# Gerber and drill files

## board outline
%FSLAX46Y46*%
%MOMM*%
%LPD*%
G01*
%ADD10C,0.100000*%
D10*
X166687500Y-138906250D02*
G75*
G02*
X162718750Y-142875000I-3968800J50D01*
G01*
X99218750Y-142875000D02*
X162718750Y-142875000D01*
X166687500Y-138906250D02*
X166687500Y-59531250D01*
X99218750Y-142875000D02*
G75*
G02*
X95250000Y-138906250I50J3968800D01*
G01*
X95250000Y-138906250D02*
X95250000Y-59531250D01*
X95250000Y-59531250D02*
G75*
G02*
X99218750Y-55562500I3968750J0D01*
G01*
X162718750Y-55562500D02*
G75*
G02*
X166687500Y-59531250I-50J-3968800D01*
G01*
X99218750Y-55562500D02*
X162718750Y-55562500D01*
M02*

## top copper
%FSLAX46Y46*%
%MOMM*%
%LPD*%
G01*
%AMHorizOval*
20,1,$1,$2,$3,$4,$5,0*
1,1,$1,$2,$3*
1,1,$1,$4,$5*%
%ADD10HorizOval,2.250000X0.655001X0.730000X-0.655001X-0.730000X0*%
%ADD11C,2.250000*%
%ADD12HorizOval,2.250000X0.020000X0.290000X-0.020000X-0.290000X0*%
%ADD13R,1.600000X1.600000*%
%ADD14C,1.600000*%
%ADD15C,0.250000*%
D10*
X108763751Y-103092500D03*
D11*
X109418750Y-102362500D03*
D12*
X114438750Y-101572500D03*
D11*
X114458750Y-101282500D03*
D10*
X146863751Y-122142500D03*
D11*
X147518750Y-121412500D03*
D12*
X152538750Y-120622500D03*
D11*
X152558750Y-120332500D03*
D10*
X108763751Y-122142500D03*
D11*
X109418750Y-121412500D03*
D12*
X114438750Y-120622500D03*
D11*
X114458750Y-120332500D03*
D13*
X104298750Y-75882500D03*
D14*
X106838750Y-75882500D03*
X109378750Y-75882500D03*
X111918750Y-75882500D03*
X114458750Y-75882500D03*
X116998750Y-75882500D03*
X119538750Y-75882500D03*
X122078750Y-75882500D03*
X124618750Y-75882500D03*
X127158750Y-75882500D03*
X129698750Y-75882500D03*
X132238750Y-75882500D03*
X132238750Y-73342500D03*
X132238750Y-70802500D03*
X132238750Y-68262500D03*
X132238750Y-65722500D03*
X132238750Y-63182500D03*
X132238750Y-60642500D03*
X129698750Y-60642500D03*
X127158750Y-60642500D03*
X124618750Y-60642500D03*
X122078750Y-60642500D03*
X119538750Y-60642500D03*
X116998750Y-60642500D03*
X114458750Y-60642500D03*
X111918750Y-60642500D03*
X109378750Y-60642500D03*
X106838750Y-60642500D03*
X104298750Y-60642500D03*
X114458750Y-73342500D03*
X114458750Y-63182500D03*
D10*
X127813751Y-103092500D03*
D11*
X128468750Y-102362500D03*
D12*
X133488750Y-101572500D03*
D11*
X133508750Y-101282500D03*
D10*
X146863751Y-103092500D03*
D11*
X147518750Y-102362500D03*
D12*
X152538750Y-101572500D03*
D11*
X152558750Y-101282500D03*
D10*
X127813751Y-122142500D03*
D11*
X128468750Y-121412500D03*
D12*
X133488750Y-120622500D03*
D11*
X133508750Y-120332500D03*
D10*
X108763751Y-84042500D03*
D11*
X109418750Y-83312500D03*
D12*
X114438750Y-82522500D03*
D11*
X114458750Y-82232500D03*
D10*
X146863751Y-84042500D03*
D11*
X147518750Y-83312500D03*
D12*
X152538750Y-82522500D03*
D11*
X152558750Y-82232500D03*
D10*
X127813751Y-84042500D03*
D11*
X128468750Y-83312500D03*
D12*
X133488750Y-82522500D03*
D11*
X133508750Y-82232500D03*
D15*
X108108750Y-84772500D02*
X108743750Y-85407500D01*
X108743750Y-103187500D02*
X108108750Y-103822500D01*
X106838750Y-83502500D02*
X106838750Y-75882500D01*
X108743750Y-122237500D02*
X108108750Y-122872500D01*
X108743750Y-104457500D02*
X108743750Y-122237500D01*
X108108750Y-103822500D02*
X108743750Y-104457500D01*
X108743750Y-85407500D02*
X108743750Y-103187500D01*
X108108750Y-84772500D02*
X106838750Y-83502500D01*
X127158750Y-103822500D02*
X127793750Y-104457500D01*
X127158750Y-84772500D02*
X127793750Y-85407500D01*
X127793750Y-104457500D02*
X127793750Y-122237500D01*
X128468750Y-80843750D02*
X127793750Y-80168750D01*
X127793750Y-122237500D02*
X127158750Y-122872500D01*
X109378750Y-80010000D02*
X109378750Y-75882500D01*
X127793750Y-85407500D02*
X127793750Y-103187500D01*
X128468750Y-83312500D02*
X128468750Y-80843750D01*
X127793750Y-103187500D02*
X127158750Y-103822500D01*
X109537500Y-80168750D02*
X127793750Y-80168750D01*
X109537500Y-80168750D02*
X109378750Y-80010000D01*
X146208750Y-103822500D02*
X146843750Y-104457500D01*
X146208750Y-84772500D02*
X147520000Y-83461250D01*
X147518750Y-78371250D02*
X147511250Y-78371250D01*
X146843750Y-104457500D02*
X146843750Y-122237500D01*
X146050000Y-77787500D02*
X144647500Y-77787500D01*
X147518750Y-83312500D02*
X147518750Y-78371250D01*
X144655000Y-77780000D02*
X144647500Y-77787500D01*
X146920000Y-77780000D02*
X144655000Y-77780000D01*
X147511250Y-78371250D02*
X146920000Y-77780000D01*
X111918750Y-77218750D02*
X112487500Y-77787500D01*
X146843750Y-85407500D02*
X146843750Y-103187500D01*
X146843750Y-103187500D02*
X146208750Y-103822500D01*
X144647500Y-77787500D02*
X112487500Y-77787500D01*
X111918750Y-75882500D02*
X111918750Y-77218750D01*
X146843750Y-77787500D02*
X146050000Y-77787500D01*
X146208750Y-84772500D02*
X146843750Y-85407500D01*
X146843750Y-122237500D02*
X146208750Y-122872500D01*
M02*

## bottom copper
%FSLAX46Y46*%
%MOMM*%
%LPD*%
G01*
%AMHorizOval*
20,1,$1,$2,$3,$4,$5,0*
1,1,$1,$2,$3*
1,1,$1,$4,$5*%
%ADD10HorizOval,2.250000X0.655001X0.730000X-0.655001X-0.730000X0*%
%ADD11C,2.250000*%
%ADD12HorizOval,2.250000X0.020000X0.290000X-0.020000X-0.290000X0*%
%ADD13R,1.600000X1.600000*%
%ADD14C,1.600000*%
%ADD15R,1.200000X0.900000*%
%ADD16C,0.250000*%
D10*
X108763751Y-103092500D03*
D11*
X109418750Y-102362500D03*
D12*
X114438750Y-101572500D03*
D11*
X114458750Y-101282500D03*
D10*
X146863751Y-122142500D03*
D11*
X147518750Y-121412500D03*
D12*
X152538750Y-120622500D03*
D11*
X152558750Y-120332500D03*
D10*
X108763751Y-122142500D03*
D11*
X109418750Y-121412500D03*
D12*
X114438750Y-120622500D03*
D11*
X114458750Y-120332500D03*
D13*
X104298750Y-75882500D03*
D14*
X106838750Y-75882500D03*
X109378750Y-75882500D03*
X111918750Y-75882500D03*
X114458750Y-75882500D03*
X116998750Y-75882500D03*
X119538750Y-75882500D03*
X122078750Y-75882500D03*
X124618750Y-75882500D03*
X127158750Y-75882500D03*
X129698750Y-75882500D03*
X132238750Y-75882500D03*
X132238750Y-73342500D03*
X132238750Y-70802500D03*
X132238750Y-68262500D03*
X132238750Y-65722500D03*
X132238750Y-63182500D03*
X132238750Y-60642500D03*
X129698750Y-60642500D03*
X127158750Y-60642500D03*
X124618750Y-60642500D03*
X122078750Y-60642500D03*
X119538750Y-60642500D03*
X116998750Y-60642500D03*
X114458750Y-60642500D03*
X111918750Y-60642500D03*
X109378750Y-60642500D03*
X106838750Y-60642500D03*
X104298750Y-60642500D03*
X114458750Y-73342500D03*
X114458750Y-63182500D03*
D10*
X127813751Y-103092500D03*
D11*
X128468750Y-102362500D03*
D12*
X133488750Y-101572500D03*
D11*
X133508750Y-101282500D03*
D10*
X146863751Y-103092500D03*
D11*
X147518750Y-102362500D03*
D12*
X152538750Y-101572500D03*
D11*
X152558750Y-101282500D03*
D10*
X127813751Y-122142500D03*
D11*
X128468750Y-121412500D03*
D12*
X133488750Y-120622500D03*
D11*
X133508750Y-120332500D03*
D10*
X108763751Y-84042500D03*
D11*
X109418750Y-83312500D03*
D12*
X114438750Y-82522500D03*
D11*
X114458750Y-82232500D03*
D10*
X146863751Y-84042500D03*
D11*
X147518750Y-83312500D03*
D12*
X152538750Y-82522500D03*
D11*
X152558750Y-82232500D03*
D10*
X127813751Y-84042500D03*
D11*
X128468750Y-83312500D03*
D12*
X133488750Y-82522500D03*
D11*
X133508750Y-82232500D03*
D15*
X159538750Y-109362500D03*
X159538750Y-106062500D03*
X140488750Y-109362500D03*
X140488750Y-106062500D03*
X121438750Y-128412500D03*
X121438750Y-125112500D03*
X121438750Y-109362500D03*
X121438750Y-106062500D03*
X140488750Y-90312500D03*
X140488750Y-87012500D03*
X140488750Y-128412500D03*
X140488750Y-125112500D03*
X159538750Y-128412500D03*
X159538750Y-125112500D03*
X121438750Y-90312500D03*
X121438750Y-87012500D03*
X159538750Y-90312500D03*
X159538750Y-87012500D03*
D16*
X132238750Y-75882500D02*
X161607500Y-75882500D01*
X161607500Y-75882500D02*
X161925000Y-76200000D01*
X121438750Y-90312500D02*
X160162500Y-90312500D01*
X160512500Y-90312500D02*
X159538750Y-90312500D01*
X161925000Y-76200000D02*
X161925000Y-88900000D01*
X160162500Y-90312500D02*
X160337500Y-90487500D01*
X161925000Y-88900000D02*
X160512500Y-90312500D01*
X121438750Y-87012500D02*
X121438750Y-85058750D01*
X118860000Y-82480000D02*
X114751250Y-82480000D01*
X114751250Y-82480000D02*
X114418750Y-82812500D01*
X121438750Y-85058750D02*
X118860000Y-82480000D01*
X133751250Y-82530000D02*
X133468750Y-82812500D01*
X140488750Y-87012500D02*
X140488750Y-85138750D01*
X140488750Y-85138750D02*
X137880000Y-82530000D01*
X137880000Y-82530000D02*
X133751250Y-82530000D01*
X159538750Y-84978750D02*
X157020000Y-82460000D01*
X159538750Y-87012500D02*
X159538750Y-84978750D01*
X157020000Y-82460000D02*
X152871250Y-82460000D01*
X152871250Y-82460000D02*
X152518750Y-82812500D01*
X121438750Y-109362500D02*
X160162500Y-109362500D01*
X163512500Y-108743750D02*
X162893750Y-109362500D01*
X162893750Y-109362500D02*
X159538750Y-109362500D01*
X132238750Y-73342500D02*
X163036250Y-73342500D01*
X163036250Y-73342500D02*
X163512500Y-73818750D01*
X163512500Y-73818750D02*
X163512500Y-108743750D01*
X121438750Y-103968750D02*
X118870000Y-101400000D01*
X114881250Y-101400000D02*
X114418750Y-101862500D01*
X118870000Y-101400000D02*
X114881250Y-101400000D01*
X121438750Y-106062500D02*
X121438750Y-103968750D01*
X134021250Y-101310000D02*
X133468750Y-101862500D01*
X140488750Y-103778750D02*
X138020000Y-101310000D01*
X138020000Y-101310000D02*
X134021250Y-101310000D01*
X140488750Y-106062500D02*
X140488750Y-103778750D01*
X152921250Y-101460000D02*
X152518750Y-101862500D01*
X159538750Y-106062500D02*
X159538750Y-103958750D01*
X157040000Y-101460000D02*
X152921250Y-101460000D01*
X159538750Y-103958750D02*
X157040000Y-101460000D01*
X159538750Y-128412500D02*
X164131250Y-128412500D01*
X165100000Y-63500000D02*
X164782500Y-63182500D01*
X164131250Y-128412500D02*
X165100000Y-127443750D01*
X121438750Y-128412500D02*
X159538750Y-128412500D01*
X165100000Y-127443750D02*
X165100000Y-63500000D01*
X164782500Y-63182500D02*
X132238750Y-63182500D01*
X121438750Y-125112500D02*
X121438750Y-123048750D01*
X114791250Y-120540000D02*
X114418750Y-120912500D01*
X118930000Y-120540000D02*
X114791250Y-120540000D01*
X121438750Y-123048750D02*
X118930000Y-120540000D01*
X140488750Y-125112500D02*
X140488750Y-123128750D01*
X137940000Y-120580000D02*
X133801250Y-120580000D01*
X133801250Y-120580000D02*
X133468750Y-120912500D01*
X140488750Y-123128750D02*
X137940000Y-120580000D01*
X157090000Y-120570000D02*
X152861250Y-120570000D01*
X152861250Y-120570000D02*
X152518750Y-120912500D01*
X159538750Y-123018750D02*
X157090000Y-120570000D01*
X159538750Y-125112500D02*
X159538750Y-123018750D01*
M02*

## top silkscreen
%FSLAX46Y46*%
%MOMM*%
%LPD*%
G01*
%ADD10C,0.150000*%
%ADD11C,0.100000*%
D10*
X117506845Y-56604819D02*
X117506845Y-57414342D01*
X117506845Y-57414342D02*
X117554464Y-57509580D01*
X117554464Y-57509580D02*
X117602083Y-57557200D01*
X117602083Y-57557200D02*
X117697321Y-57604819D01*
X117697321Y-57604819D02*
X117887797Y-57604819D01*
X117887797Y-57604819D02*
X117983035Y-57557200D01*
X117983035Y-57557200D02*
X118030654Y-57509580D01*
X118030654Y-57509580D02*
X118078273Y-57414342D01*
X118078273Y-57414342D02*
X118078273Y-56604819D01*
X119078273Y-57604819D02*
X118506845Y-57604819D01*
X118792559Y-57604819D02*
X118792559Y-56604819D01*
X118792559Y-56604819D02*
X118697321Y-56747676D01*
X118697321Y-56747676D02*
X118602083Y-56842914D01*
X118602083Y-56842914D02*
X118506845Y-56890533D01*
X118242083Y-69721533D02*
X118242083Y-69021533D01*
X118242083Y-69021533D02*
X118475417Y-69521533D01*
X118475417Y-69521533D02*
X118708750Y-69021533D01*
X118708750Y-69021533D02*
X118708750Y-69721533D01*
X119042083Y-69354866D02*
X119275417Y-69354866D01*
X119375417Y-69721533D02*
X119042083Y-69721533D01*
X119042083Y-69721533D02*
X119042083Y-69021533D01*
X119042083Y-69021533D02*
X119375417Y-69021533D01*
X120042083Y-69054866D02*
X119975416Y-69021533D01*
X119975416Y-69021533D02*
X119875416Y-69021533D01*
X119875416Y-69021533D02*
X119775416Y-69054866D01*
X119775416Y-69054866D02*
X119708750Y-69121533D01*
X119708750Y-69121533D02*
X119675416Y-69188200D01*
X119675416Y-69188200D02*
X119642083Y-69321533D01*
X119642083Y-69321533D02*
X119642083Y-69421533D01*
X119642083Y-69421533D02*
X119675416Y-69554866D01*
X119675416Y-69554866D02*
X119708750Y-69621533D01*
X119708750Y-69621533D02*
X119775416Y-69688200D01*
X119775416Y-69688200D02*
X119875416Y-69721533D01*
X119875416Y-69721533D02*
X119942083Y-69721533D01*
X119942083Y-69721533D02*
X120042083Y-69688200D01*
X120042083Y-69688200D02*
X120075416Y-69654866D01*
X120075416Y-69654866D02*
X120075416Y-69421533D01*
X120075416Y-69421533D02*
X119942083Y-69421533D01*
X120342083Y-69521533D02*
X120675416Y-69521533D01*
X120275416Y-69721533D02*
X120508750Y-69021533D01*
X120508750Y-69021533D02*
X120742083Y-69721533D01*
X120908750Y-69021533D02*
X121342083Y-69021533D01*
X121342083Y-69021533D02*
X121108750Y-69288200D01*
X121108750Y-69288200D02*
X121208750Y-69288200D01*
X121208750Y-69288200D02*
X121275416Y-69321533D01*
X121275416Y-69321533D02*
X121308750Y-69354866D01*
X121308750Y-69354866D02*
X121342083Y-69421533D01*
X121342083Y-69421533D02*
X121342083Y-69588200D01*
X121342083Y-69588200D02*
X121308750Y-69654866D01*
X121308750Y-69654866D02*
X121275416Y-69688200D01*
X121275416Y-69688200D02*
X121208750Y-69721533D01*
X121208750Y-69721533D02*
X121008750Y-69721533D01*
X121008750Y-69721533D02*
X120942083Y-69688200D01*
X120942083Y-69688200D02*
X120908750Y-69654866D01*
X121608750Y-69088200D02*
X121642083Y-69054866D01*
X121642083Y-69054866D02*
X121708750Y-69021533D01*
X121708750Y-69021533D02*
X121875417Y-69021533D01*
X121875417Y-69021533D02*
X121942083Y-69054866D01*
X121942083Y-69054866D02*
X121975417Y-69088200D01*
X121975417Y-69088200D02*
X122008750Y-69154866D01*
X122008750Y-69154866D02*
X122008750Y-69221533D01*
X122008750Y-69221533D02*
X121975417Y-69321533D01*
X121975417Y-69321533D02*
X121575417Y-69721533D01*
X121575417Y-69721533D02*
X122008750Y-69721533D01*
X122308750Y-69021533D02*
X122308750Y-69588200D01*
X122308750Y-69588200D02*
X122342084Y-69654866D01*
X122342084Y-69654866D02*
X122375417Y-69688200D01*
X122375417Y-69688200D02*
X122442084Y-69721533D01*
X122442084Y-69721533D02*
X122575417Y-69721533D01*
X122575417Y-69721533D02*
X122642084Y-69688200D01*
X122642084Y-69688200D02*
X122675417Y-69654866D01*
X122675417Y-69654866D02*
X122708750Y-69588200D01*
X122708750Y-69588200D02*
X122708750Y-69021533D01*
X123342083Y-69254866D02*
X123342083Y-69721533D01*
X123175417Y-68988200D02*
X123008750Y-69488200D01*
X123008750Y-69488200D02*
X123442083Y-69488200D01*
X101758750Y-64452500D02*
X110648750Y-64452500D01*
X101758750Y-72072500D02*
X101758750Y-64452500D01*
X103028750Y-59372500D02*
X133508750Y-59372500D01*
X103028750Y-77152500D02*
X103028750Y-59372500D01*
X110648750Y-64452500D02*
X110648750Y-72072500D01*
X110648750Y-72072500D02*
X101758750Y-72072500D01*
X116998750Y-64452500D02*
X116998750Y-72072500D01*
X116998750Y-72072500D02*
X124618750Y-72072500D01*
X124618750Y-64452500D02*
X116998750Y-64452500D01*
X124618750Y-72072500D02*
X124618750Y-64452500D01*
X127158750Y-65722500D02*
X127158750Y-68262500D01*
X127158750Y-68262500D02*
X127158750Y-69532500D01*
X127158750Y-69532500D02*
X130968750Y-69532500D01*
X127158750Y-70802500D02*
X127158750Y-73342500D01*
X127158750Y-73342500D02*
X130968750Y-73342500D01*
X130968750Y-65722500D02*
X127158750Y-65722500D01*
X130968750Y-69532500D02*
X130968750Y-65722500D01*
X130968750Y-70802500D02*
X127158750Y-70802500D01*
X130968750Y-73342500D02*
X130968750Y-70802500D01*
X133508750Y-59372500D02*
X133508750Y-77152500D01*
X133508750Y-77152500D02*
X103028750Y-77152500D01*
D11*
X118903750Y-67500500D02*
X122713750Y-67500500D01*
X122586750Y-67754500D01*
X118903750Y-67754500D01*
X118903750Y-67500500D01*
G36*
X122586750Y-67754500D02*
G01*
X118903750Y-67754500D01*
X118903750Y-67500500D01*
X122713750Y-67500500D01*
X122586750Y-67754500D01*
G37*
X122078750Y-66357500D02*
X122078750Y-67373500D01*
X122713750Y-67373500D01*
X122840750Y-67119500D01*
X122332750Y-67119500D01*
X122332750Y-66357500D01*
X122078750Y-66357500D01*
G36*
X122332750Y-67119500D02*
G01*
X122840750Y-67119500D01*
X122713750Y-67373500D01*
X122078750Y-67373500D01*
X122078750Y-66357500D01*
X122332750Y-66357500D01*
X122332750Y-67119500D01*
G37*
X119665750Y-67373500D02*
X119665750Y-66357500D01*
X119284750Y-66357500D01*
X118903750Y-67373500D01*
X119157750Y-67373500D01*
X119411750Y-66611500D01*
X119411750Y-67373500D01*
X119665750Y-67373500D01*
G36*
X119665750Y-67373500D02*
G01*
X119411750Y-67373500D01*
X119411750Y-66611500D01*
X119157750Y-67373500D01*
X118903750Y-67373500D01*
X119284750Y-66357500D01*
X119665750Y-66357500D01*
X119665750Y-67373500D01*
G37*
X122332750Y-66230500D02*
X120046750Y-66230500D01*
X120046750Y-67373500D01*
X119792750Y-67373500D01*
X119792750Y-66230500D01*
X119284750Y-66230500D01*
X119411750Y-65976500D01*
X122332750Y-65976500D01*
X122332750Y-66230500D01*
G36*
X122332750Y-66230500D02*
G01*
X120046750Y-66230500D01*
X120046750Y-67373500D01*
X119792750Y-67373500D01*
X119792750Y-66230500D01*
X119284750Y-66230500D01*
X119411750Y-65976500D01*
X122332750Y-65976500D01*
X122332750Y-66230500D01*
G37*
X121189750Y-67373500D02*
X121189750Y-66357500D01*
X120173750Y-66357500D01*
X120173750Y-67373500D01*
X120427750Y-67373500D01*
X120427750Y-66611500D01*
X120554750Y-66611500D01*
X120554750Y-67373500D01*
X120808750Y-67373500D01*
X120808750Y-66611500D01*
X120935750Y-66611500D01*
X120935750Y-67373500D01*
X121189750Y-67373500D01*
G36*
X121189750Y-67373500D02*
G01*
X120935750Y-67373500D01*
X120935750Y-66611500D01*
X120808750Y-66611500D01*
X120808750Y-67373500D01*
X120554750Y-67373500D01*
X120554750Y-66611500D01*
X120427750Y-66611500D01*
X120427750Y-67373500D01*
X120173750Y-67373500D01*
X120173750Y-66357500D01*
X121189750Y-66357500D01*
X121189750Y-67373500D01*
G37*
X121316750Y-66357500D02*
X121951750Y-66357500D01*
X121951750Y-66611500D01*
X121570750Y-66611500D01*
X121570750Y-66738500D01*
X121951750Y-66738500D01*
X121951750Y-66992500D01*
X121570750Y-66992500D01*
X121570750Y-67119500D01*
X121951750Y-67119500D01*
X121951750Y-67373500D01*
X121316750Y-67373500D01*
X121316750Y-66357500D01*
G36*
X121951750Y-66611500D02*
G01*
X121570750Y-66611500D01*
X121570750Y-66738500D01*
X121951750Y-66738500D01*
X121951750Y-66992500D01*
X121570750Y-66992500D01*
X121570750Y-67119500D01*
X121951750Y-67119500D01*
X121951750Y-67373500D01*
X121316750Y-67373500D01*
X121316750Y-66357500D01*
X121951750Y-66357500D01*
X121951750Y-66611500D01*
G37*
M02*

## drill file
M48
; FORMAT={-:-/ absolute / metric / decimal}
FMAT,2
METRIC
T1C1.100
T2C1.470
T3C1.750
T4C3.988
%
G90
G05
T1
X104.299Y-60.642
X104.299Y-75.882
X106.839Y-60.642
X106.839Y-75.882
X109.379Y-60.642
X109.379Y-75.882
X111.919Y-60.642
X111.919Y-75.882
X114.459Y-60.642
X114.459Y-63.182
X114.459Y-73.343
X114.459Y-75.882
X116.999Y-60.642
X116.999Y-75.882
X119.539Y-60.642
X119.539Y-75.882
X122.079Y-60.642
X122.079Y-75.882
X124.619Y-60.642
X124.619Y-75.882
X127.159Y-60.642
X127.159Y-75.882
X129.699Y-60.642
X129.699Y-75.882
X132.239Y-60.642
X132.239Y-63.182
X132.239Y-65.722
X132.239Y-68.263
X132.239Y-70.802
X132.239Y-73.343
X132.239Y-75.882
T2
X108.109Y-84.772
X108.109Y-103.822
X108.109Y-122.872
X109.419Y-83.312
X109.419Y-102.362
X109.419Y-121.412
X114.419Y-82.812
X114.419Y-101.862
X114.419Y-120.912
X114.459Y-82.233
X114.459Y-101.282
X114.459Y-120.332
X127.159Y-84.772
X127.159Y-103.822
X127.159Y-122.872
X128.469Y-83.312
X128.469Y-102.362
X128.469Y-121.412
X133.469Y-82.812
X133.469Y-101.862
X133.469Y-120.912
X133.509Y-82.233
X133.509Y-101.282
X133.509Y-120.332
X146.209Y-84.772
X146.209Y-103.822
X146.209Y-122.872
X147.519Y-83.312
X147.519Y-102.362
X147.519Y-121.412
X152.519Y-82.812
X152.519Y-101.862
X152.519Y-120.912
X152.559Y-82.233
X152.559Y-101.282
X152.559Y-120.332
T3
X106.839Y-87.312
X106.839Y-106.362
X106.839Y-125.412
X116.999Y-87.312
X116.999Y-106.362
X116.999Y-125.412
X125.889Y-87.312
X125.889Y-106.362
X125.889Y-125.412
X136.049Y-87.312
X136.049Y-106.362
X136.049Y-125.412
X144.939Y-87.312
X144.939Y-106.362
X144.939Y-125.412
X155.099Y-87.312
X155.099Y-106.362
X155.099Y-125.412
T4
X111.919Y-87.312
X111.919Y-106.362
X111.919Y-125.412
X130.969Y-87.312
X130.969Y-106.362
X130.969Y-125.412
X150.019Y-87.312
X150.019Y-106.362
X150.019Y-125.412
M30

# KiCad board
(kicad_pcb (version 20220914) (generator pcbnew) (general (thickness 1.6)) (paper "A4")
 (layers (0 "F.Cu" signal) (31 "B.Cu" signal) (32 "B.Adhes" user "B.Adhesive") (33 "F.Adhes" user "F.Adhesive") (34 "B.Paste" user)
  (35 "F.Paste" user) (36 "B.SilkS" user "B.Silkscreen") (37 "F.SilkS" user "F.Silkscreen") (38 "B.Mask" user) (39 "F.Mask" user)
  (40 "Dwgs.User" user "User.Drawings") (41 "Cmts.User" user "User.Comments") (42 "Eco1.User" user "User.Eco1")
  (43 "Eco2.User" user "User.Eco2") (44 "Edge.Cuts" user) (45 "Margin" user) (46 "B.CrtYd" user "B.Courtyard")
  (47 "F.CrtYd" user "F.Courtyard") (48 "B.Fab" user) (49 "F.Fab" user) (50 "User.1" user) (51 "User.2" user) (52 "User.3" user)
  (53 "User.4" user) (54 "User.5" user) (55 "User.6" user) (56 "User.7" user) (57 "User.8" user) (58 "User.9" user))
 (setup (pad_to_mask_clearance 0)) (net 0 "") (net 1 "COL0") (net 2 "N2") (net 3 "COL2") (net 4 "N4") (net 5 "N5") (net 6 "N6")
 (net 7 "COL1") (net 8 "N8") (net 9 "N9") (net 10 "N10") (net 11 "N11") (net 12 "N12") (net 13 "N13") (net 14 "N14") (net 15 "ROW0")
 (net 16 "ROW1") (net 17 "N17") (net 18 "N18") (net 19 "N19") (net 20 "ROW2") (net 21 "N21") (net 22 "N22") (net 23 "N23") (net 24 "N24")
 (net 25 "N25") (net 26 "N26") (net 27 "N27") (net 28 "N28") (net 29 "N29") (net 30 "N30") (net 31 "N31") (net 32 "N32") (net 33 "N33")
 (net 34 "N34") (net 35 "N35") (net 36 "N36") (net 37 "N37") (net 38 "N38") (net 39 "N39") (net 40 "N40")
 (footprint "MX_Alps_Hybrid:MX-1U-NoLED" (layer "F.Cu") (at 111.91875 106.3625)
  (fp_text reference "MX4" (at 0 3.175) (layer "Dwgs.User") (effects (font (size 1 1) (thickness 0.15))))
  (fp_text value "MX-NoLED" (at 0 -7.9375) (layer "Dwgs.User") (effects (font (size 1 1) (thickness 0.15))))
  (pad "" np_thru_hole circle (at -5.08 0 48.0996) (size 1.75 1.75) (drill 1.75) (layers *.Cu *.Mask))
  (pad "" np_thru_hole circle (at 0 0) (size 3.9878 3.9878) (drill 3.9878) (layers *.Cu *.Mask))
  (pad "" np_thru_hole circle (at 5.08 0 48.0996) (size 1.75 1.75) (drill 1.75) (layers *.Cu *.Mask))
  (pad "1" thru_hole oval (at -3.81 -2.54 48.0996) (size 4.211556 2.25) (drill 1.47 (offset 0.980778 0)) (layers *.Cu "B.Mask")
   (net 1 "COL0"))
  (pad "1" thru_hole circle (at -2.5 -4) (size 2.25 2.25) (drill 1.47) (layers *.Cu "B.Mask") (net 1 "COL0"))
  (pad "2" thru_hole oval (at 2.5 -4.5 86.0548) (size 2.831378 2.25) (drill 1.47 (offset 0.290689 0)) (layers *.Cu "B.Mask") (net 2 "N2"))
  (pad "2" thru_hole circle (at 2.54 -5.08) (size 2.25 2.25) (drill 1.47) (layers *.Cu "B.Mask") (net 2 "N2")))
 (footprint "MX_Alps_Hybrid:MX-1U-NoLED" (layer "F.Cu") (at 150.01875 125.4125)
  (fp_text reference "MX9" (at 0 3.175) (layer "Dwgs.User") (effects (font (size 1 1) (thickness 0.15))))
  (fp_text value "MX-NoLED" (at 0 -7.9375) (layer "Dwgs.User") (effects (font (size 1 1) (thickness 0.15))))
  (pad "" np_thru_hole circle (at -5.08 0 48.0996) (size 1.75 1.75) (drill 1.75) (layers *.Cu *.Mask))
  (pad "" np_thru_hole circle (at 0 0) (size 3.9878 3.9878) (drill 3.9878) (layers *.Cu *.Mask))
  (pad "" np_thru_hole circle (at 5.08 0 48.0996) (size 1.75 1.75) (drill 1.75) (layers *.Cu *.Mask))
  (pad "1" thru_hole oval (at -3.81 -2.54 48.0996) (size 4.211556 2.25) (drill 1.47 (offset 0.980778 0)) (layers *.Cu "B.Mask")
   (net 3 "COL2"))
  (pad "1" thru_hole circle (at -2.5 -4) (size 2.25 2.25) (drill 1.47) (layers *.Cu "B.Mask") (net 3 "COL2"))
  (pad "2" thru_hole oval (at 2.5 -4.5 86.0548) (size 2.831378 2.25) (drill 1.47 (offset 0.290689 0)) (layers *.Cu "B.Mask") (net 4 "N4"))
  (pad "2" thru_hole circle (at 2.54 -5.08) (size 2.25 2.25) (drill 1.47) (layers *.Cu "B.Mask") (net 4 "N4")))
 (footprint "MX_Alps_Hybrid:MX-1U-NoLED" (layer "F.Cu") (at 111.91875 125.4125)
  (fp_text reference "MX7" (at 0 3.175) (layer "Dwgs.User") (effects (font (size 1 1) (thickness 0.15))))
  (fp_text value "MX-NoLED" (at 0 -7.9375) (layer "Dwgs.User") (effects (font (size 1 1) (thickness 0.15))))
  (pad "" np_thru_hole circle (at -5.08 0 48.0996) (size 1.75 1.75) (drill 1.75) (layers *.Cu *.Mask))
  (pad "" np_thru_hole circle (at 0 0) (size 3.9878 3.9878) (drill 3.9878) (layers *.Cu *.Mask))
  (pad "" np_thru_hole circle (at 5.08 0 48.0996) (size 1.75 1.75) (drill 1.75) (layers *.Cu *.Mask))
  (pad "1" thru_hole oval (at -3.81 -2.54 48.0996) (size 4.211556 2.25) (drill 1.47 (offset 0.980778 0)) (layers *.Cu "B.Mask")
   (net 1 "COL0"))
  (pad "1" thru_hole circle (at -2.5 -4) (size 2.25 2.25) (drill 1.47) (layers *.Cu "B.Mask") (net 1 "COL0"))
  (pad "2" thru_hole oval (at 2.5 -4.5 86.0548) (size 2.831378 2.25) (drill 1.47 (offset 0.290689 0)) (layers *.Cu "B.Mask") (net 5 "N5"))
  (pad "2" thru_hole circle (at 2.54 -5.08) (size 2.25 2.25) (drill 1.47) (layers *.Cu "B.Mask") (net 5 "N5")))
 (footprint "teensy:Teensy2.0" (layer "F.Cu") (at 118.26875 68.2625)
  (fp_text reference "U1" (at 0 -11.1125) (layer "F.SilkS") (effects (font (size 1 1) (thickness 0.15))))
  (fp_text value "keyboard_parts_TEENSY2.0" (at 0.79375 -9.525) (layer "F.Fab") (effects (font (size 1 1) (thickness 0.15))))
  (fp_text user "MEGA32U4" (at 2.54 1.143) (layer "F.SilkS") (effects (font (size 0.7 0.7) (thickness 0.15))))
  (fp_line (start -16.51 -3.81) (end -7.62 -3.81) (stroke (width 0.15) (type solid)) (layer "F.SilkS"))
  (fp_line (start -16.51 3.81) (end -16.51 -3.81) (stroke (width 0.15) (type solid)) (layer "F.SilkS"))
  (fp_line (start -15.24 -8.89) (end 15.24 -8.89) (stroke (width 0.15) (type solid)) (layer "F.SilkS"))
  (fp_line (start -15.24 8.89) (end -15.24 -8.89) (stroke (width 0.15) (type solid)) (layer "F.SilkS"))
  (fp_line (start -7.62 -3.81) (end -7.62 3.81) (stroke (width 0.15) (type solid)) (layer "F.SilkS"))
  (fp_line (start -7.62 3.81) (end -16.51 3.81) (stroke (width 0.15) (type solid)) (layer "F.SilkS"))
  (fp_line (start -1.27 -3.81) (end -1.27 3.81) (stroke (width 0.15) (type solid)) (layer "F.SilkS"))
  (fp_line (start -1.27 3.81) (end 6.35 3.81) (stroke (width 0.15) (type solid)) (layer "F.SilkS"))
  (fp_line (start 6.35 -3.81) (end -1.27 -3.81) (stroke (width 0.15) (type solid)) (layer "F.SilkS"))
  (fp_line (start 6.35 3.81) (end 6.35 -3.81) (stroke (width 0.15) (type solid)) (layer "F.SilkS"))
  (fp_line (start 8.89 -2.54) (end 8.89 0) (stroke (width 0.15) (type solid)) (layer "F.SilkS"))
  (fp_line (start 8.89 0) (end 8.89 1.27) (stroke (width 0.15) (type solid)) (layer "F.SilkS"))
  (fp_line (start 8.89 1.27) (end 12.7 1.27) (stroke (width 0.15) (type solid)) (layer "F.SilkS"))
  (fp_line (start 8.89 2.54) (end 8.89 5.08) (stroke (width 0.15) (type solid)) (layer "F.SilkS"))
  (fp_line (start 8.89 5.08) (end 12.7 5.08) (stroke (width 0.15) (type solid)) (layer "F.SilkS"))
  (fp_line (start 12.7 -2.54) (end 8.89 -2.54) (stroke (width 0.15) (type solid)) (layer "F.SilkS"))
  (fp_line (start 12.7 1.27) (end 12.7 -2.54) (stroke (width 0.15) (type solid)) (layer "F.SilkS"))
  (fp_line (start 12.7 2.54) (end 8.89 2.54) (stroke (width 0.15) (type solid)) (layer "F.SilkS"))
  (fp_line (start 12.7 5.08) (end 12.7 2.54) (stroke (width 0.15) (type solid)) (layer "F.SilkS"))
  (fp_line (start 15.24 -8.89) (end 15.24 8.89) (stroke (width 0.15) (type solid)) (layer "F.SilkS"))
  (fp_line (start 15.24 8.89) (end -15.24 8.89) (stroke (width 0.15) (type solid)) (layer "F.SilkS"))
  (fp_poly
   (pts (xy 0.635 -0.762) (xy 4.445 -0.762) (xy 4.318 -0.508) (xy 0.635 -0.508)) (stroke (width 0.1) (type solid)) (fill solid)
   (layer "F.SilkS"))
  (fp_poly
   (pts (xy 3.81 -1.905) (xy 3.81 -0.889) (xy 4.445 -0.889) (xy 4.572 -1.143) (xy 4.064 -1.143) (xy 4.064 -1.905))
   (stroke (width 0.1) (type solid)) (fill solid) (layer "F.SilkS"))
  (fp_poly
   (pts (xy 1.397 -0.889) (xy 1.397 -1.905) (xy 1.016 -1.905) (xy 0.635 -0.889) (xy 0.889 -0.889) (xy 1.143 -1.651) (xy 1.143 -0.889))
   (stroke (width 0.1) (type solid)) (fill solid) (layer "F.SilkS"))
  (fp_poly
   (pts (xy 4.064 -2.032) (xy 1.778 -2.032) (xy 1.778 -0.889) (xy 1.524 -0.889) (xy 1.524 -2.032) (xy 1.016 -2.032) (xy 1.143 -2.286)
    (xy 4.064 -2.286))
   (stroke (width 0.1) (type solid)) (fill solid) (layer "F.SilkS"))
  (fp_poly
   (pts (xy 2.921 -0.889) (xy 2.921 -1.905) (xy 1.905 -1.905) (xy 1.905 -0.889) (xy 2.159 -0.889) (xy 2.159 -1.651) (xy 2.286 -1.651)
    (xy 2.286 -0.889) (xy 2.54 -0.889) (xy 2.54 -1.651) (xy 2.667 -1.651) (xy 2.667 -0.889))
   (stroke (width 0.1) (type solid)) (fill solid) (layer "F.SilkS"))
  (fp_poly
   (pts (xy 3.048 -1.905) (xy 3.683 -1.905) (xy 3.683 -1.651) (xy 3.302 -1.651) (xy 3.302 -1.524) (xy 3.683 -1.524) (xy 3.683 -1.27)
    (xy 3.302 -1.27) (xy 3.302 -1.143) (xy 3.683 -1.143) (xy 3.683 -0.889) (xy 3.048 -0.889))
   (stroke (width 0.1) (type solid)) (fill solid) (layer "F.SilkS"))
  (pad "1" thru_hole rect (at -13.97 7.62) (size 1.6 1.6) (drill 1.1) (layers *.Cu *.Mask) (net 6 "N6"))
  (pad "2" thru_hole circle (at -11.43 7.62) (size 1.6 1.6) (drill 1.1) (layers *.Cu *.Mask) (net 1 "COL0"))
  (pad "3" thru_hole circle (at -8.89 7.62) (size 1.6 1.6) (drill 1.1) (layers *.Cu *.Mask) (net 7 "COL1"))
  (pad "4" thru_hole circle (at -6.35 7.62) (size 1.6 1.6) (drill 1.1) (layers *.Cu *.Mask) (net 3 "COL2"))
  (pad "5" thru_hole circle (at -3.81 7.62) (size 1.6 1.6) (drill 1.1) (layers *.Cu *.Mask) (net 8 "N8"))
  (pad "6" thru_hole circle (at -1.27 7.62) (size 1.6 1.6) (drill 1.1) (layers *.Cu *.Mask) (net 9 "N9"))
  (pad "7" thru_hole circle (at 1.27 7.62) (size 1.6 1.6) (drill 1.1) (layers *.Cu *.Mask) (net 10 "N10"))
  (pad "8" thru_hole circle (at 3.81 7.62) (size 1.6 1.6) (drill 1.1) (layers *.Cu *.Mask) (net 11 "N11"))
  (pad "9" thru_hole circle (at 6.35 7.62) (size 1.6 1.6) (drill 1.1) (layers *.Cu *.Mask) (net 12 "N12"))
  (pad "10" thru_hole circle (at 8.89 7.62) (size 1.6 1.6) (drill 1.1) (layers *.Cu *.Mask) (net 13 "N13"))
  (pad "11" thru_hole circle (at 11.43 7.62) (size 1.6 1.6) (drill 1.1) (layers *.Cu *.Mask) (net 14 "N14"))
  (pad "12" thru_hole circle (at 13.97 7.62) (size 1.6 1.6) (drill 1.1) (layers *.Cu *.Mask) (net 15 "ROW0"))
  (pad "13" thru_hole circle (at 13.97 5.08) (size 1.6 1.6) (drill 1.1) (layers *.Cu *.Mask) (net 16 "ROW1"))
  (pad "14" thru_hole circle (at 13.97 2.54) (size 1.6 1.6) (drill 1.1) (layers *.Cu *.Mask) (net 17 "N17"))
  (pad "15" thru_hole circle (at 13.97 0) (size 1.6 1.6) (drill 1.1) (layers *.Cu *.Mask) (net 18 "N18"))
  (pad "16" thru_hole circle (at 13.97 -2.54) (size 1.6 1.6) (drill 1.1) (layers *.Cu *.Mask) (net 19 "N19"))
  (pad "17" thru_hole circle (at 13.97 -5.08) (size 1.6 1.6) (drill 1.1) (layers *.Cu *.Mask) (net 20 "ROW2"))
  (pad "18" thru_hole circle (at 13.97 -7.62) (size 1.6 1.6) (drill 1.1) (layers *.Cu *.Mask) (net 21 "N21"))
  (pad "19" thru_hole circle (at 11.43 -7.62) (size 1.6 1.6) (drill 1.1) (layers *.Cu *.Mask) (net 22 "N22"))
  (pad "20" thru_hole circle (at 8.89 -7.62) (size 1.6 1.6) (drill 1.1) (layers *.Cu *.Mask) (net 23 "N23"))
  (pad "21" thru_hole circle (at 6.35 -7.62) (size 1.6 1.6) (drill 1.1) (layers *.Cu *.Mask) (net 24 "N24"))
  (pad "22" thru_hole circle (at 3.81 -7.62) (size 1.6 1.6) (drill 1.1) (layers *.Cu *.Mask) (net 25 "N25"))
  (pad "23" thru_hole circle (at 1.27 -7.62) (size 1.6 1.6) (drill 1.1) (layers *.Cu *.Mask) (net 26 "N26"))
  (pad "24" thru_hole circle (at -1.27 -7.62) (size 1.6 1.6) (drill 1.1) (layers *.Cu *.Mask) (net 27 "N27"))
  (pad "25" thru_hole circle (at -3.81 -7.62) (size 1.6 1.6) (drill 1.1) (layers *.Cu *.Mask) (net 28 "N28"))
  (pad "26" thru_hole circle (at -6.35 -7.62) (size 1.6 1.6) (drill 1.1) (layers *.Cu *.Mask) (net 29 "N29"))
  (pad "27" thru_hole circle (at -8.89 -7.62) (size 1.6 1.6) (drill 1.1) (layers *.Cu *.Mask) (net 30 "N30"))
  (pad "28" thru_hole circle (at -11.43 -7.62) (size 1.6 1.6) (drill 1.1) (layers *.Cu *.Mask) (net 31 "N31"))
  (pad "29" thru_hole circle (at -13.97 -7.62) (size 1.6 1.6) (drill 1.1) (layers *.Cu *.Mask) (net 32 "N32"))
  (pad "30" thru_hole circle (at -3.81 5.08) (size 1.6 1.6) (drill 1.1) (layers *.Cu *.Mask) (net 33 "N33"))
  (pad "31" thru_hole circle (at -3.81 -5.08) (size 1.6 1.6) (drill 1.1) (layers *.Cu *.Mask) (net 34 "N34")))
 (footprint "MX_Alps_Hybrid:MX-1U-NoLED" (layer "F.Cu") (at 130.96875 106.3625)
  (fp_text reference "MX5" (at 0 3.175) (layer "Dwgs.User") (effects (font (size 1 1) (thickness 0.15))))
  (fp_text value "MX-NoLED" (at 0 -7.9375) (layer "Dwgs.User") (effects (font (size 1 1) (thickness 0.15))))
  (pad "" np_thru_hole circle (at -5.08 0 48.0996) (size 1.75 1.75) (drill 1.75) (layers *.Cu *.Mask))
  (pad "" np_thru_hole circle (at 0 0) (size 3.9878 3.9878) (drill 3.9878) (layers *.Cu *.Mask))
  (pad "" np_thru_hole circle (at 5.08 0 48.0996) (size 1.75 1.75) (drill 1.75) (layers *.Cu *.Mask))
  (pad "1" thru_hole oval (at -3.81 -2.54 48.0996) (size 4.211556 2.25) (drill 1.47 (offset 0.980778 0)) (layers *.Cu "B.Mask")
   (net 7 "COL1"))
  (pad "1" thru_hole circle (at -2.5 -4) (size 2.25 2.25) (drill 1.47) (layers *.Cu "B.Mask") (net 7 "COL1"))
  (pad "2" thru_hole oval (at 2.5 -4.5 86.0548) (size 2.831378 2.25) (drill 1.47 (offset 0.290689 0)) (layers *.Cu "B.Mask") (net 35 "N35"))
  (pad "2" thru_hole circle (at 2.54 -5.08) (size 2.25 2.25) (drill 1.47) (layers *.Cu "B.Mask") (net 35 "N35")))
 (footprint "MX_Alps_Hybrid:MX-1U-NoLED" (layer "F.Cu") (at 150.01875 106.3625)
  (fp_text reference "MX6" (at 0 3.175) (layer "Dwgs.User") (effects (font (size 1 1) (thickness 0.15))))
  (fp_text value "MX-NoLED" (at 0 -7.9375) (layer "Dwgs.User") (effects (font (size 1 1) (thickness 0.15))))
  (pad "" np_thru_hole circle (at -5.08 0 48.0996) (size 1.75 1.75) (drill 1.75) (layers *.Cu *.Mask))
  (pad "" np_thru_hole circle (at 0 0) (size 3.9878 3.9878) (drill 3.9878) (layers *.Cu *.Mask))
  (pad "" np_thru_hole circle (at 5.08 0 48.0996) (size 1.75 1.75) (drill 1.75) (layers *.Cu *.Mask))
  (pad "1" thru_hole oval (at -3.81 -2.54 48.0996) (size 4.211556 2.25) (drill 1.47 (offset 0.980778 0)) (layers *.Cu "B.Mask")
   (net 3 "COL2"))
  (pad "1" thru_hole circle (at -2.5 -4) (size 2.25 2.25) (drill 1.47) (layers *.Cu "B.Mask") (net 3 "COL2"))
  (pad "2" thru_hole oval (at 2.5 -4.5 86.0548) (size 2.831378 2.25) (drill 1.47 (offset 0.290689 0)) (layers *.Cu "B.Mask") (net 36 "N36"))
  (pad "2" thru_hole circle (at 2.54 -5.08) (size 2.25 2.25) (drill 1.47) (layers *.Cu "B.Mask") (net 36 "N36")))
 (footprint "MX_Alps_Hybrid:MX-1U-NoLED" (layer "F.Cu") (at 130.96875 125.4125)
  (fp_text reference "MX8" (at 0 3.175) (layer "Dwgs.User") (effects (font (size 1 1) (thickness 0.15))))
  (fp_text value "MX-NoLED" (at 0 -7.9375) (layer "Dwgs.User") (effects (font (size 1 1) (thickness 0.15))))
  (pad "" np_thru_hole circle (at -5.08 0 48.0996) (size 1.75 1.75) (drill 1.75) (layers *.Cu *.Mask))
  (pad "" np_thru_hole circle (at 0 0) (size 3.9878 3.9878) (drill 3.9878) (layers *.Cu *.Mask))
  (pad "" np_thru_hole circle (at 5.08 0 48.0996) (size 1.75 1.75) (drill 1.75) (layers *.Cu *.Mask))
  (pad "1" thru_hole oval (at -3.81 -2.54 48.0996) (size 4.211556 2.25) (drill 1.47 (offset 0.980778 0)) (layers *.Cu "B.Mask")
   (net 7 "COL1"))
  (pad "1" thru_hole circle (at -2.5 -4) (size 2.25 2.25) (drill 1.47) (layers *.Cu "B.Mask") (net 7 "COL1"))
  (pad "2" thru_hole oval (at 2.5 -4.5 86.0548) (size 2.831378 2.25) (drill 1.47 (offset 0.290689 0)) (layers *.Cu "B.Mask") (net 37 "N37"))
  (pad "2" thru_hole circle (at 2.54 -5.08) (size 2.25 2.25) (drill 1.47) (layers *.Cu "B.Mask") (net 37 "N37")))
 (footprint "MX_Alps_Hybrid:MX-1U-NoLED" (layer "F.Cu") (at 111.91875 87.3125)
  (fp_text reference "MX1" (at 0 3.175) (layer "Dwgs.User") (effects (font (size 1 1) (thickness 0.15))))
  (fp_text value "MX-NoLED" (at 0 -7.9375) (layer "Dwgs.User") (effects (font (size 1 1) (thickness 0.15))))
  (pad "" np_thru_hole circle (at -5.08 0 48.0996) (size 1.75 1.75) (drill 1.75) (layers *.Cu *.Mask))
  (pad "" np_thru_hole circle (at 0 0) (size 3.9878 3.9878) (drill 3.9878) (layers *.Cu *.Mask))
  (pad "" np_thru_hole circle (at 5.08 0 48.0996) (size 1.75 1.75) (drill 1.75) (layers *.Cu *.Mask))
  (pad "1" thru_hole oval (at -3.81 -2.54 48.0996) (size 4.211556 2.25) (drill 1.47 (offset 0.980778 0)) (layers *.Cu "B.Mask")
   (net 1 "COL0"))
  (pad "1" thru_hole circle (at -2.5 -4) (size 2.25 2.25) (drill 1.47) (layers *.Cu "B.Mask") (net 1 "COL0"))
  (pad "2" thru_hole oval (at 2.5 -4.5 86.0548) (size 2.831378 2.25) (drill 1.47 (offset 0.290689 0)) (layers *.Cu "B.Mask") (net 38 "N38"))
  (pad "2" thru_hole circle (at 2.54 -5.08) (size 2.25 2.25) (drill 1.47) (layers *.Cu "B.Mask") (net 38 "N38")))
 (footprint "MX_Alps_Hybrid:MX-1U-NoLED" (layer "F.Cu") (at 150.01875 87.3125)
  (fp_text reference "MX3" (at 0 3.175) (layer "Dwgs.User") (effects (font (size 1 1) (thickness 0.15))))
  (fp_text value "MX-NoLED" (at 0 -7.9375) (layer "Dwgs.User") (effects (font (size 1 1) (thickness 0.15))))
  (pad "" np_thru_hole circle (at -5.08 0 48.0996) (size 1.75 1.75) (drill 1.75) (layers *.Cu *.Mask))
  (pad "" np_thru_hole circle (at 0 0) (size 3.9878 3.9878) (drill 3.9878) (layers *.Cu *.Mask))
  (pad "" np_thru_hole circle (at 5.08 0 48.0996) (size 1.75 1.75) (drill 1.75) (layers *.Cu *.Mask))
  (pad "1" thru_hole oval (at -3.81 -2.54 48.0996) (size 4.211556 2.25) (drill 1.47 (offset 0.980778 0)) (layers *.Cu "B.Mask")
   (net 3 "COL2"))
  (pad "1" thru_hole circle (at -2.5 -4) (size 2.25 2.25) (drill 1.47) (layers *.Cu "B.Mask") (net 3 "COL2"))
  (pad "2" thru_hole oval (at 2.5 -4.5 86.0548) (size 2.831378 2.25) (drill 1.47 (offset 0.290689 0)) (layers *.Cu "B.Mask") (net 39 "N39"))
  (pad "2" thru_hole circle (at 2.54 -5.08) (size 2.25 2.25) (drill 1.47) (layers *.Cu "B.Mask") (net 39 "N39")))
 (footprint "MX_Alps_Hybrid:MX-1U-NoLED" (layer "F.Cu") (at 130.96875 87.3125)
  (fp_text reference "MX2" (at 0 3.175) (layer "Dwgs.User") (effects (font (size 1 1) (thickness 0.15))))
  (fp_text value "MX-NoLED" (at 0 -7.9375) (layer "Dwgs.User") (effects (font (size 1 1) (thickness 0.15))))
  (pad "" np_thru_hole circle (at -5.08 0 48.0996) (size 1.75 1.75) (drill 1.75) (layers *.Cu *.Mask))
  (pad "" np_thru_hole circle (at 0 0) (size 3.9878 3.9878) (drill 3.9878) (layers *.Cu *.Mask))
  (pad "" np_thru_hole circle (at 5.08 0 48.0996) (size 1.75 1.75) (drill 1.75) (layers *.Cu *.Mask))
  (pad "1" thru_hole oval (at -3.81 -2.54 48.0996) (size 4.211556 2.25) (drill 1.47 (offset 0.980778 0)) (layers *.Cu "B.Mask")
   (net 7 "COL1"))
  (pad "1" thru_hole circle (at -2.5 -4) (size 2.25 2.25) (drill 1.47) (layers *.Cu "B.Mask") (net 7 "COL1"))
  (pad "2" thru_hole oval (at 2.5 -4.5 86.0548) (size 2.831378 2.25) (drill 1.47 (offset 0.290689 0)) (layers *.Cu "B.Mask") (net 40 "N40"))
  (pad "2" thru_hole circle (at 2.54 -5.08) (size 2.25 2.25) (drill 1.47) (layers *.Cu "B.Mask") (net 40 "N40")))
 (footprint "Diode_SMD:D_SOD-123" (layer "B.Cu") (at 159.53875 107.7125 90)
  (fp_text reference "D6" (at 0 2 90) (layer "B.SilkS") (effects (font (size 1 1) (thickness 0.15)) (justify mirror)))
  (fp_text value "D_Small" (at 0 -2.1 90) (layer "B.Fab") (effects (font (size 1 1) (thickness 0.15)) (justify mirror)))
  (pad "1" smd rect (at -1.65 0 90) (size 0.9 1.2) (layers "B.Cu" "B.Paste" "B.Mask") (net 16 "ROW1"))
  (pad "2" smd rect (at 1.65 0 90) (size 0.9 1.2) (layers "B.Cu" "B.Paste" "B.Mask") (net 36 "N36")))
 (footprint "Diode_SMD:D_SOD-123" (layer "B.Cu") (at 140.48875 107.7125 90)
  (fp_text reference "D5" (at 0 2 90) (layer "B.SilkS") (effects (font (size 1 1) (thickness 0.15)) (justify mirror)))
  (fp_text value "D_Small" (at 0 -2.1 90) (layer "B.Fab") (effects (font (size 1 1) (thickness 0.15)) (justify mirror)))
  (pad "1" smd rect (at -1.65 0 90) (size 0.9 1.2) (layers "B.Cu" "B.Paste" "B.Mask") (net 16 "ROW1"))
  (pad "2" smd rect (at 1.65 0 90) (size 0.9 1.2) (layers "B.Cu" "B.Paste" "B.Mask") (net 35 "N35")))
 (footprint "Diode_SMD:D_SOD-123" (layer "B.Cu") (at 121.43875 126.7625 90)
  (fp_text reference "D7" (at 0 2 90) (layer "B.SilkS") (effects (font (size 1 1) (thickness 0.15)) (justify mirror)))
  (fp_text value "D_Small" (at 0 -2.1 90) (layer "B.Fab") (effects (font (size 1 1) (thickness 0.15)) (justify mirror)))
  (pad "1" smd rect (at -1.65 0 90) (size 0.9 1.2) (layers "B.Cu" "B.Paste" "B.Mask") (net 20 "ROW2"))
  (pad "2" smd rect (at 1.65 0 90) (size 0.9 1.2) (layers "B.Cu" "B.Paste" "B.Mask") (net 5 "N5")))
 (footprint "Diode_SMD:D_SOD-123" (layer "B.Cu") (at 121.43875 107.7125 90)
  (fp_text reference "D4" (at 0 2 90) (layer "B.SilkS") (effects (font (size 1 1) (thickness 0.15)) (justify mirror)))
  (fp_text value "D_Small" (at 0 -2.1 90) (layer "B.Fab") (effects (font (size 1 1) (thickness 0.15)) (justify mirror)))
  (pad "1" smd rect (at -1.65 0 90) (size 0.9 1.2) (layers "B.Cu" "B.Paste" "B.Mask") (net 16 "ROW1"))
  (pad "2" smd rect (at 1.65 0 90) (size 0.9 1.2) (layers "B.Cu" "B.Paste" "B.Mask") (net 2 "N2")))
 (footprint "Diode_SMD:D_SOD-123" (layer "B.Cu") (at 140.48875 88.6625 90)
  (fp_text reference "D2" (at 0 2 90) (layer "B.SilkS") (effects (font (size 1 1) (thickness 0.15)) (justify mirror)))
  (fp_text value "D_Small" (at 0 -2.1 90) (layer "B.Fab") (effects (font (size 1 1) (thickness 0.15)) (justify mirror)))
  (pad "1" smd rect (at -1.65 0 90) (size 0.9 1.2) (layers "B.Cu" "B.Paste" "B.Mask") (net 15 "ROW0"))
  (pad "2" smd rect (at 1.65 0 90) (size 0.9 1.2) (layers "B.Cu" "B.Paste" "B.Mask") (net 40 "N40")))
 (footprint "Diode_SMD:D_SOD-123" (layer "B.Cu") (at 140.48875 126.7625 90)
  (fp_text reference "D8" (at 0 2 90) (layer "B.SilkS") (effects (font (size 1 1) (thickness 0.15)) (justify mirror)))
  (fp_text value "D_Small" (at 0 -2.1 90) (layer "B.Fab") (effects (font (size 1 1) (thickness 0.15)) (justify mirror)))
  (pad "1" smd rect (at -1.65 0 90) (size 0.9 1.2) (layers "B.Cu" "B.Paste" "B.Mask") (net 20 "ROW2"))
  (pad "2" smd rect (at 1.65 0 90) (size 0.9 1.2) (layers "B.Cu" "B.Paste" "B.Mask") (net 37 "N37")))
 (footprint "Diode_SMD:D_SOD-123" (layer "B.Cu") (at 159.53875 126.7625 90)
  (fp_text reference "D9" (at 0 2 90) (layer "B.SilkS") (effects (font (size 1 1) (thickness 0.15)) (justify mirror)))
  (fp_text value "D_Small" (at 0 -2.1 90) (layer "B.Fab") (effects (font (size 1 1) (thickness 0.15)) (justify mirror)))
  (pad "1" smd rect (at -1.65 0 90) (size 0.9 1.2) (layers "B.Cu" "B.Paste" "B.Mask") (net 20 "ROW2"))
  (pad "2" smd rect (at 1.65 0 90) (size 0.9 1.2) (layers "B.Cu" "B.Paste" "B.Mask") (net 4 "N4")))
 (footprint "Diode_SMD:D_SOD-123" (layer "B.Cu") (at 121.43875 88.6625 90)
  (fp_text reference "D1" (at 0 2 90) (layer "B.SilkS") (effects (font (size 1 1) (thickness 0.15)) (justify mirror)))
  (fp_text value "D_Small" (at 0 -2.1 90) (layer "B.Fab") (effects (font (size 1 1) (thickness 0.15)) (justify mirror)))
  (pad "1" smd rect (at -1.65 0 90) (size 0.9 1.2) (layers "B.Cu" "B.Paste" "B.Mask") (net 15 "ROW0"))
  (pad "2" smd rect (at 1.65 0 90) (size 0.9 1.2) (layers "B.Cu" "B.Paste" "B.Mask") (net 38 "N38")))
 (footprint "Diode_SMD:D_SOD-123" (layer "B.Cu") (at 159.53875 88.6625 90)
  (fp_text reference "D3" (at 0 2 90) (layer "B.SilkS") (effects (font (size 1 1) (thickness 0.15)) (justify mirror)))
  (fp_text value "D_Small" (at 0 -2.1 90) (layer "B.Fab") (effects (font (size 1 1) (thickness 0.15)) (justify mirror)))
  (pad "1" smd rect (at -1.65 0 90) (size 0.9 1.2) (layers "B.Cu" "B.Paste" "B.Mask") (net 15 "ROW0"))
  (pad "2" smd rect (at 1.65 0 90) (size 0.9 1.2) (layers "B.Cu" "B.Paste" "B.Mask") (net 39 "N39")))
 (gr_arc (start 166.6875 138.90625) (mid 165.52508 141.71258) (end 162.71875 142.875) (stroke (width 0.1) (type default))
  (layer "Edge.Cuts"))
 (gr_line (start 99.21875 142.875) (end 162.71875 142.875) (stroke (width 0.1) (type default)) (layer "Edge.Cuts"))
 (gr_line (start 166.6875 138.90625) (end 166.6875 59.53125) (stroke (width 0.1) (type default)) (layer "Edge.Cuts"))
 (gr_arc (start 99.21875 142.875) (mid 96.41242 141.71258) (end 95.25 138.90625) (stroke (width 0.1) (type default)) (layer "Edge.Cuts"))
 (gr_line (start 95.25 138.90625) (end 95.25 59.53125) (stroke (width 0.1) (type default)) (layer "Edge.Cuts"))
 (gr_arc (start 95.25 59.53125) (mid 96.41242 56.72492) (end 99.21875 55.5625) (stroke (width 0.1) (type default)) (layer "Edge.Cuts"))
 (gr_arc (start 162.71875 55.5625) (mid 165.52508 56.72492) (end 166.6875 59.53125) (stroke (width 0.1) (type default)) (layer "Edge.Cuts"))
 (gr_line (start 99.21875 55.5625) (end 162.71875 55.5625) (stroke (width 0.1) (type default)) (layer "Edge.Cuts"))
 (segment (start 132.23875 75.8825) (end 161.6075 75.8825) (width 0.25) (layer "B.Cu") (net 15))
 (segment (start 161.6075 75.8825) (end 161.925 76.2) (width 0.25) (layer "B.Cu") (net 15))
 (segment (start 121.43875 90.3125) (end 160.1625 90.3125) (width 0.25) (layer "B.Cu") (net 15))
 (segment (start 160.5125 90.3125) (end 159.53875 90.3125) (width 0.25) (layer "B.Cu") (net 15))
 (segment (start 161.925 76.2) (end 161.925 88.9) (width 0.25) (layer "B.Cu") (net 15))
 (segment (start 160.1625 90.3125) (end 160.3375 90.4875) (width 0.25) (layer "B.Cu") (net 15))
 (segment (start 161.925 88.9) (end 160.5125 90.3125) (width 0.25) (layer "B.Cu") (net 15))
 (segment (start 121.43875 87.0125) (end 121.43875 85.05875) (width 0.25) (layer "B.Cu") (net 38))
 (segment (start 118.86 82.48) (end 114.75125 82.48) (width 0.25) (layer "B.Cu") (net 38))
 (segment (start 114.75125 82.48) (end 114.41875 82.8125) (width 0.25) (layer "B.Cu") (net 38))
 (segment (start 121.43875 85.05875) (end 118.86 82.48) (width 0.25) (layer "B.Cu") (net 38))
 (segment (start 133.75125 82.53) (end 133.46875 82.8125) (width 0.25) (layer "B.Cu") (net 40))
 (segment (start 140.48875 87.0125) (end 140.48875 85.13875) (width 0.25) (layer "B.Cu") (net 40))
 (segment (start 140.48875 85.13875) (end 137.88 82.53) (width 0.25) (layer "B.Cu") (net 40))
 (segment (start 137.88 82.53) (end 133.75125 82.53) (width 0.25) (layer "B.Cu") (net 40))
 (segment (start 159.53875 84.97875) (end 157.02 82.46) (width 0.25) (layer "B.Cu") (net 39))
 (segment (start 159.53875 87.0125) (end 159.53875 84.97875) (width 0.25) (layer "B.Cu") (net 39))
 (segment (start 157.02 82.46) (end 152.87125 82.46) (width 0.25) (layer "B.Cu") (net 39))
 (segment (start 152.87125 82.46) (end 152.51875 82.8125) (width 0.25) (layer "B.Cu") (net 39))
 (segment (start 121.43875 109.3625) (end 160.1625 109.3625) (width 0.25) (layer "B.Cu") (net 16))
 (segment (start 163.5125 108.74375) (end 162.89375 109.3625) (width 0.25) (layer "B.Cu") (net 16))
 (segment (start 162.89375 109.3625) (end 159.53875 109.3625) (width 0.25) (layer "B.Cu") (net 16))
 (segment (start 132.23875 73.3425) (end 163.03625 73.3425) (width 0.25) (layer "B.Cu") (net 16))
 (segment (start 163.03625 73.3425) (end 163.5125 73.81875) (width 0.25) (layer "B.Cu") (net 16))
 (segment (start 163.5125 73.81875) (end 163.5125 108.74375) (width 0.25) (layer "B.Cu") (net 16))
 (segment (start 121.43875 103.96875) (end 118.87 101.4) (width 0.25) (layer "B.Cu") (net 2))
 (segment (start 114.88125 101.4) (end 114.41875 101.8625) (width 0.25) (layer "B.Cu") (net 2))
 (segment (start 118.87 101.4) (end 114.88125 101.4) (width 0.25) (layer "B.Cu") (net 2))
 (segment (start 121.43875 106.0625) (end 121.43875 103.96875) (width 0.25) (layer "B.Cu") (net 2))
 (segment (start 134.02125 101.31) (end 133.46875 101.8625) (width 0.25) (layer "B.Cu") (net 35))
 (segment (start 140.48875 103.77875) (end 138.02 101.31) (width 0.25) (layer "B.Cu") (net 35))
 (segment (start 138.02 101.31) (end 134.02125 101.31) (width 0.25) (layer "B.Cu") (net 35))
 (segment (start 140.48875 106.0625) (end 140.48875 103.77875) (width 0.25) (layer "B.Cu") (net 35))
 (segment (start 152.92125 101.46) (end 152.51875 101.8625) (width 0.25) (layer "B.Cu") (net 36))
 (segment (start 159.53875 106.0625) (end 159.53875 103.95875) (width 0.25) (layer "B.Cu") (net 36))
 (segment (start 157.04 101.46) (end 152.92125 101.46) (width 0.25) (layer "B.Cu") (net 36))
 (segment (start 159.53875 103.95875) (end 157.04 101.46) (width 0.25) (layer "B.Cu") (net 36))
 (segment (start 159.53875 128.4125) (end 164.13125 128.4125) (width 0.25) (layer "B.Cu") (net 20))
 (segment (start 165.1 63.5) (end 164.7825 63.1825) (width 0.25) (layer "B.Cu") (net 20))
 (segment (start 164.13125 128.4125) (end 165.1 127.44375) (width 0.25) (layer "B.Cu") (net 20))
 (segment (start 121.43875 128.4125) (end 159.53875 128.4125) (width 0.25) (layer "B.Cu") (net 20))
 (segment (start 165.1 127.44375) (end 165.1 63.5) (width 0.25) (layer "B.Cu") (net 20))
 (segment (start 164.7825 63.1825) (end 132.23875 63.1825) (width 0.25) (layer "B.Cu") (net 20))
 (segment (start 121.43875 125.1125) (end 121.43875 123.04875) (width 0.25) (layer "B.Cu") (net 5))
 (segment (start 114.79125 120.54) (end 114.41875 120.9125) (width 0.25) (layer "B.Cu") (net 5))
 (segment (start 118.93 120.54) (end 114.79125 120.54) (width 0.25) (layer "B.Cu") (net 5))
 (segment (start 121.43875 123.04875) (end 118.93 120.54) (width 0.25) (layer "B.Cu") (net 5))
 (segment (start 140.48875 125.1125) (end 140.48875 123.12875) (width 0.25) (layer "B.Cu") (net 37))
 (segment (start 137.94 120.58) (end 133.80125 120.58) (width 0.25) (layer "B.Cu") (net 37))
 (segment (start 133.80125 120.58) (end 133.46875 120.9125) (width 0.25) (layer "B.Cu") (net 37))
 (segment (start 140.48875 123.12875) (end 137.94 120.58) (width 0.25) (layer "B.Cu") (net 37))
 (segment (start 157.09 120.57) (end 152.86125 120.57) (width 0.25) (layer "B.Cu") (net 4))
 (segment (start 152.86125 120.57) (end 152.51875 120.9125) (width 0.25) (layer "B.Cu") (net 4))
 (segment (start 159.53875 123.01875) (end 157.09 120.57) (width 0.25) (layer "B.Cu") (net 4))
 (segment (start 159.53875 125.1125) (end 159.53875 123.01875) (width 0.25) (layer "B.Cu") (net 4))
 (segment (start 108.10875 84.7725) (end 108.74375 85.4075) (width 0.25) (layer "F.Cu") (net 1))
 (segment (start 108.74375 103.1875) (end 108.10875 103.8225) (width 0.25) (layer "F.Cu") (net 1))
 (segment (start 106.83875 83.5025) (end 106.83875 75.8825) (width 0.25) (layer "F.Cu") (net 1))
 (segment (start 108.74375 122.2375) (end 108.10875 122.8725) (width 0.25) (layer "F.Cu") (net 1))
 (segment (start 108.74375 104.4575) (end 108.74375 122.2375) (width 0.25) (layer "F.Cu") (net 1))
 (segment (start 108.10875 103.8225) (end 108.74375 104.4575) (width 0.25) (layer "F.Cu") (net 1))
 (segment (start 108.74375 85.4075) (end 108.74375 103.1875) (width 0.25) (layer "F.Cu") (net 1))
 (segment (start 108.10875 84.7725) (end 106.83875 83.5025) (width 0.25) (layer "F.Cu") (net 1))
 (segment (start 127.15875 103.8225) (end 127.79375 104.4575) (width 0.25) (layer "F.Cu") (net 7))
 (segment (start 127.15875 84.7725) (end 127.79375 85.4075) (width 0.25) (layer "F.Cu") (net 7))
 (segment (start 127.79375 104.4575) (end 127.79375 122.2375) (width 0.25) (layer "F.Cu") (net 7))
 (segment (start 128.46875 80.84375) (end 127.79375 80.16875) (width 0.25) (layer "F.Cu") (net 7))
 (segment (start 127.79375 122.2375) (end 127.15875 122.8725) (width 0.25) (layer "F.Cu") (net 7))
 (segment (start 109.37875 80.01) (end 109.37875 75.8825) (width 0.25) (layer "F.Cu") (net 7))
 (segment (start 127.79375 85.4075) (end 127.79375 103.1875) (width 0.25) (layer "F.Cu") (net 7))
 (segment (start 128.46875 83.3125) (end 128.46875 80.84375) (width 0.25) (layer "F.Cu") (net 7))
 (segment (start 127.79375 103.1875) (end 127.15875 103.8225) (width 0.25) (layer "F.Cu") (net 7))
 (segment (start 109.5375 80.16875) (end 127.79375 80.16875) (width 0.25) (layer "F.Cu") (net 7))
 (segment (start 109.5375 80.16875) (end 109.37875 80.01) (width 0.25) (layer "F.Cu") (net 7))
 (segment (start 146.20875 103.8225) (end 146.84375 104.4575) (width 0.25) (layer "F.Cu") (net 3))
 (segment (start 146.20875 84.7725) (end 147.52 83.46125) (width 0.25) (layer "F.Cu") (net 3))
 (segment (start 147.51875 78.37125) (end 147.51125 78.37125) (width 0.25) (layer "F.Cu") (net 3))
 (segment (start 146.84375 104.4575) (end 146.84375 122.2375) (width 0.25) (layer "F.Cu") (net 3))
 (segment (start 146.05 77.7875) (end 144.6475 77.7875) (width 0.25) (layer "F.Cu") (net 3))
 (segment (start 147.51875 83.3125) (end 147.51875 78.37125) (width 0.25) (layer "F.Cu") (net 3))
 (segment (start 144.655 77.78) (end 144.6475 77.7875) (width 0.25) (layer "F.Cu") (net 3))
 (segment (start 146.92 77.78) (end 144.655 77.78) (width 0.25) (layer "F.Cu") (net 3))
 (segment (start 147.51125 78.37125) (end 146.92 77.78) (width 0.25) (layer "F.Cu") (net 3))
 (segment (start 111.91875 77.21875) (end 112.4875 77.7875) (width 0.25) (layer "F.Cu") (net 3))
 (segment (start 146.84375 85.4075) (end 146.84375 103.1875) (width 0.25) (layer "F.Cu") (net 3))
 (segment (start 146.84375 103.1875) (end 146.20875 103.8225) (width 0.25) (layer "F.Cu") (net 3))
 (segment (start 144.6475 77.7875) (end 112.4875 77.7875) (width 0.25) (layer "F.Cu") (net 3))
 (segment (start 111.91875 75.8825) (end 111.91875 77.21875) (width 0.25) (layer "F.Cu") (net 3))
 (segment (start 146.84375 77.7875) (end 146.05 77.7875) (width 0.25) (layer "F.Cu") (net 3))
 (segment (start 146.20875 84.7725) (end 146.84375 85.4075) (width 0.25) (layer "F.Cu") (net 3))
 (segment (start 146.84375 122.2375) (end 146.20875 122.8725) (width 0.25) (layer "F.Cu") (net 3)))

